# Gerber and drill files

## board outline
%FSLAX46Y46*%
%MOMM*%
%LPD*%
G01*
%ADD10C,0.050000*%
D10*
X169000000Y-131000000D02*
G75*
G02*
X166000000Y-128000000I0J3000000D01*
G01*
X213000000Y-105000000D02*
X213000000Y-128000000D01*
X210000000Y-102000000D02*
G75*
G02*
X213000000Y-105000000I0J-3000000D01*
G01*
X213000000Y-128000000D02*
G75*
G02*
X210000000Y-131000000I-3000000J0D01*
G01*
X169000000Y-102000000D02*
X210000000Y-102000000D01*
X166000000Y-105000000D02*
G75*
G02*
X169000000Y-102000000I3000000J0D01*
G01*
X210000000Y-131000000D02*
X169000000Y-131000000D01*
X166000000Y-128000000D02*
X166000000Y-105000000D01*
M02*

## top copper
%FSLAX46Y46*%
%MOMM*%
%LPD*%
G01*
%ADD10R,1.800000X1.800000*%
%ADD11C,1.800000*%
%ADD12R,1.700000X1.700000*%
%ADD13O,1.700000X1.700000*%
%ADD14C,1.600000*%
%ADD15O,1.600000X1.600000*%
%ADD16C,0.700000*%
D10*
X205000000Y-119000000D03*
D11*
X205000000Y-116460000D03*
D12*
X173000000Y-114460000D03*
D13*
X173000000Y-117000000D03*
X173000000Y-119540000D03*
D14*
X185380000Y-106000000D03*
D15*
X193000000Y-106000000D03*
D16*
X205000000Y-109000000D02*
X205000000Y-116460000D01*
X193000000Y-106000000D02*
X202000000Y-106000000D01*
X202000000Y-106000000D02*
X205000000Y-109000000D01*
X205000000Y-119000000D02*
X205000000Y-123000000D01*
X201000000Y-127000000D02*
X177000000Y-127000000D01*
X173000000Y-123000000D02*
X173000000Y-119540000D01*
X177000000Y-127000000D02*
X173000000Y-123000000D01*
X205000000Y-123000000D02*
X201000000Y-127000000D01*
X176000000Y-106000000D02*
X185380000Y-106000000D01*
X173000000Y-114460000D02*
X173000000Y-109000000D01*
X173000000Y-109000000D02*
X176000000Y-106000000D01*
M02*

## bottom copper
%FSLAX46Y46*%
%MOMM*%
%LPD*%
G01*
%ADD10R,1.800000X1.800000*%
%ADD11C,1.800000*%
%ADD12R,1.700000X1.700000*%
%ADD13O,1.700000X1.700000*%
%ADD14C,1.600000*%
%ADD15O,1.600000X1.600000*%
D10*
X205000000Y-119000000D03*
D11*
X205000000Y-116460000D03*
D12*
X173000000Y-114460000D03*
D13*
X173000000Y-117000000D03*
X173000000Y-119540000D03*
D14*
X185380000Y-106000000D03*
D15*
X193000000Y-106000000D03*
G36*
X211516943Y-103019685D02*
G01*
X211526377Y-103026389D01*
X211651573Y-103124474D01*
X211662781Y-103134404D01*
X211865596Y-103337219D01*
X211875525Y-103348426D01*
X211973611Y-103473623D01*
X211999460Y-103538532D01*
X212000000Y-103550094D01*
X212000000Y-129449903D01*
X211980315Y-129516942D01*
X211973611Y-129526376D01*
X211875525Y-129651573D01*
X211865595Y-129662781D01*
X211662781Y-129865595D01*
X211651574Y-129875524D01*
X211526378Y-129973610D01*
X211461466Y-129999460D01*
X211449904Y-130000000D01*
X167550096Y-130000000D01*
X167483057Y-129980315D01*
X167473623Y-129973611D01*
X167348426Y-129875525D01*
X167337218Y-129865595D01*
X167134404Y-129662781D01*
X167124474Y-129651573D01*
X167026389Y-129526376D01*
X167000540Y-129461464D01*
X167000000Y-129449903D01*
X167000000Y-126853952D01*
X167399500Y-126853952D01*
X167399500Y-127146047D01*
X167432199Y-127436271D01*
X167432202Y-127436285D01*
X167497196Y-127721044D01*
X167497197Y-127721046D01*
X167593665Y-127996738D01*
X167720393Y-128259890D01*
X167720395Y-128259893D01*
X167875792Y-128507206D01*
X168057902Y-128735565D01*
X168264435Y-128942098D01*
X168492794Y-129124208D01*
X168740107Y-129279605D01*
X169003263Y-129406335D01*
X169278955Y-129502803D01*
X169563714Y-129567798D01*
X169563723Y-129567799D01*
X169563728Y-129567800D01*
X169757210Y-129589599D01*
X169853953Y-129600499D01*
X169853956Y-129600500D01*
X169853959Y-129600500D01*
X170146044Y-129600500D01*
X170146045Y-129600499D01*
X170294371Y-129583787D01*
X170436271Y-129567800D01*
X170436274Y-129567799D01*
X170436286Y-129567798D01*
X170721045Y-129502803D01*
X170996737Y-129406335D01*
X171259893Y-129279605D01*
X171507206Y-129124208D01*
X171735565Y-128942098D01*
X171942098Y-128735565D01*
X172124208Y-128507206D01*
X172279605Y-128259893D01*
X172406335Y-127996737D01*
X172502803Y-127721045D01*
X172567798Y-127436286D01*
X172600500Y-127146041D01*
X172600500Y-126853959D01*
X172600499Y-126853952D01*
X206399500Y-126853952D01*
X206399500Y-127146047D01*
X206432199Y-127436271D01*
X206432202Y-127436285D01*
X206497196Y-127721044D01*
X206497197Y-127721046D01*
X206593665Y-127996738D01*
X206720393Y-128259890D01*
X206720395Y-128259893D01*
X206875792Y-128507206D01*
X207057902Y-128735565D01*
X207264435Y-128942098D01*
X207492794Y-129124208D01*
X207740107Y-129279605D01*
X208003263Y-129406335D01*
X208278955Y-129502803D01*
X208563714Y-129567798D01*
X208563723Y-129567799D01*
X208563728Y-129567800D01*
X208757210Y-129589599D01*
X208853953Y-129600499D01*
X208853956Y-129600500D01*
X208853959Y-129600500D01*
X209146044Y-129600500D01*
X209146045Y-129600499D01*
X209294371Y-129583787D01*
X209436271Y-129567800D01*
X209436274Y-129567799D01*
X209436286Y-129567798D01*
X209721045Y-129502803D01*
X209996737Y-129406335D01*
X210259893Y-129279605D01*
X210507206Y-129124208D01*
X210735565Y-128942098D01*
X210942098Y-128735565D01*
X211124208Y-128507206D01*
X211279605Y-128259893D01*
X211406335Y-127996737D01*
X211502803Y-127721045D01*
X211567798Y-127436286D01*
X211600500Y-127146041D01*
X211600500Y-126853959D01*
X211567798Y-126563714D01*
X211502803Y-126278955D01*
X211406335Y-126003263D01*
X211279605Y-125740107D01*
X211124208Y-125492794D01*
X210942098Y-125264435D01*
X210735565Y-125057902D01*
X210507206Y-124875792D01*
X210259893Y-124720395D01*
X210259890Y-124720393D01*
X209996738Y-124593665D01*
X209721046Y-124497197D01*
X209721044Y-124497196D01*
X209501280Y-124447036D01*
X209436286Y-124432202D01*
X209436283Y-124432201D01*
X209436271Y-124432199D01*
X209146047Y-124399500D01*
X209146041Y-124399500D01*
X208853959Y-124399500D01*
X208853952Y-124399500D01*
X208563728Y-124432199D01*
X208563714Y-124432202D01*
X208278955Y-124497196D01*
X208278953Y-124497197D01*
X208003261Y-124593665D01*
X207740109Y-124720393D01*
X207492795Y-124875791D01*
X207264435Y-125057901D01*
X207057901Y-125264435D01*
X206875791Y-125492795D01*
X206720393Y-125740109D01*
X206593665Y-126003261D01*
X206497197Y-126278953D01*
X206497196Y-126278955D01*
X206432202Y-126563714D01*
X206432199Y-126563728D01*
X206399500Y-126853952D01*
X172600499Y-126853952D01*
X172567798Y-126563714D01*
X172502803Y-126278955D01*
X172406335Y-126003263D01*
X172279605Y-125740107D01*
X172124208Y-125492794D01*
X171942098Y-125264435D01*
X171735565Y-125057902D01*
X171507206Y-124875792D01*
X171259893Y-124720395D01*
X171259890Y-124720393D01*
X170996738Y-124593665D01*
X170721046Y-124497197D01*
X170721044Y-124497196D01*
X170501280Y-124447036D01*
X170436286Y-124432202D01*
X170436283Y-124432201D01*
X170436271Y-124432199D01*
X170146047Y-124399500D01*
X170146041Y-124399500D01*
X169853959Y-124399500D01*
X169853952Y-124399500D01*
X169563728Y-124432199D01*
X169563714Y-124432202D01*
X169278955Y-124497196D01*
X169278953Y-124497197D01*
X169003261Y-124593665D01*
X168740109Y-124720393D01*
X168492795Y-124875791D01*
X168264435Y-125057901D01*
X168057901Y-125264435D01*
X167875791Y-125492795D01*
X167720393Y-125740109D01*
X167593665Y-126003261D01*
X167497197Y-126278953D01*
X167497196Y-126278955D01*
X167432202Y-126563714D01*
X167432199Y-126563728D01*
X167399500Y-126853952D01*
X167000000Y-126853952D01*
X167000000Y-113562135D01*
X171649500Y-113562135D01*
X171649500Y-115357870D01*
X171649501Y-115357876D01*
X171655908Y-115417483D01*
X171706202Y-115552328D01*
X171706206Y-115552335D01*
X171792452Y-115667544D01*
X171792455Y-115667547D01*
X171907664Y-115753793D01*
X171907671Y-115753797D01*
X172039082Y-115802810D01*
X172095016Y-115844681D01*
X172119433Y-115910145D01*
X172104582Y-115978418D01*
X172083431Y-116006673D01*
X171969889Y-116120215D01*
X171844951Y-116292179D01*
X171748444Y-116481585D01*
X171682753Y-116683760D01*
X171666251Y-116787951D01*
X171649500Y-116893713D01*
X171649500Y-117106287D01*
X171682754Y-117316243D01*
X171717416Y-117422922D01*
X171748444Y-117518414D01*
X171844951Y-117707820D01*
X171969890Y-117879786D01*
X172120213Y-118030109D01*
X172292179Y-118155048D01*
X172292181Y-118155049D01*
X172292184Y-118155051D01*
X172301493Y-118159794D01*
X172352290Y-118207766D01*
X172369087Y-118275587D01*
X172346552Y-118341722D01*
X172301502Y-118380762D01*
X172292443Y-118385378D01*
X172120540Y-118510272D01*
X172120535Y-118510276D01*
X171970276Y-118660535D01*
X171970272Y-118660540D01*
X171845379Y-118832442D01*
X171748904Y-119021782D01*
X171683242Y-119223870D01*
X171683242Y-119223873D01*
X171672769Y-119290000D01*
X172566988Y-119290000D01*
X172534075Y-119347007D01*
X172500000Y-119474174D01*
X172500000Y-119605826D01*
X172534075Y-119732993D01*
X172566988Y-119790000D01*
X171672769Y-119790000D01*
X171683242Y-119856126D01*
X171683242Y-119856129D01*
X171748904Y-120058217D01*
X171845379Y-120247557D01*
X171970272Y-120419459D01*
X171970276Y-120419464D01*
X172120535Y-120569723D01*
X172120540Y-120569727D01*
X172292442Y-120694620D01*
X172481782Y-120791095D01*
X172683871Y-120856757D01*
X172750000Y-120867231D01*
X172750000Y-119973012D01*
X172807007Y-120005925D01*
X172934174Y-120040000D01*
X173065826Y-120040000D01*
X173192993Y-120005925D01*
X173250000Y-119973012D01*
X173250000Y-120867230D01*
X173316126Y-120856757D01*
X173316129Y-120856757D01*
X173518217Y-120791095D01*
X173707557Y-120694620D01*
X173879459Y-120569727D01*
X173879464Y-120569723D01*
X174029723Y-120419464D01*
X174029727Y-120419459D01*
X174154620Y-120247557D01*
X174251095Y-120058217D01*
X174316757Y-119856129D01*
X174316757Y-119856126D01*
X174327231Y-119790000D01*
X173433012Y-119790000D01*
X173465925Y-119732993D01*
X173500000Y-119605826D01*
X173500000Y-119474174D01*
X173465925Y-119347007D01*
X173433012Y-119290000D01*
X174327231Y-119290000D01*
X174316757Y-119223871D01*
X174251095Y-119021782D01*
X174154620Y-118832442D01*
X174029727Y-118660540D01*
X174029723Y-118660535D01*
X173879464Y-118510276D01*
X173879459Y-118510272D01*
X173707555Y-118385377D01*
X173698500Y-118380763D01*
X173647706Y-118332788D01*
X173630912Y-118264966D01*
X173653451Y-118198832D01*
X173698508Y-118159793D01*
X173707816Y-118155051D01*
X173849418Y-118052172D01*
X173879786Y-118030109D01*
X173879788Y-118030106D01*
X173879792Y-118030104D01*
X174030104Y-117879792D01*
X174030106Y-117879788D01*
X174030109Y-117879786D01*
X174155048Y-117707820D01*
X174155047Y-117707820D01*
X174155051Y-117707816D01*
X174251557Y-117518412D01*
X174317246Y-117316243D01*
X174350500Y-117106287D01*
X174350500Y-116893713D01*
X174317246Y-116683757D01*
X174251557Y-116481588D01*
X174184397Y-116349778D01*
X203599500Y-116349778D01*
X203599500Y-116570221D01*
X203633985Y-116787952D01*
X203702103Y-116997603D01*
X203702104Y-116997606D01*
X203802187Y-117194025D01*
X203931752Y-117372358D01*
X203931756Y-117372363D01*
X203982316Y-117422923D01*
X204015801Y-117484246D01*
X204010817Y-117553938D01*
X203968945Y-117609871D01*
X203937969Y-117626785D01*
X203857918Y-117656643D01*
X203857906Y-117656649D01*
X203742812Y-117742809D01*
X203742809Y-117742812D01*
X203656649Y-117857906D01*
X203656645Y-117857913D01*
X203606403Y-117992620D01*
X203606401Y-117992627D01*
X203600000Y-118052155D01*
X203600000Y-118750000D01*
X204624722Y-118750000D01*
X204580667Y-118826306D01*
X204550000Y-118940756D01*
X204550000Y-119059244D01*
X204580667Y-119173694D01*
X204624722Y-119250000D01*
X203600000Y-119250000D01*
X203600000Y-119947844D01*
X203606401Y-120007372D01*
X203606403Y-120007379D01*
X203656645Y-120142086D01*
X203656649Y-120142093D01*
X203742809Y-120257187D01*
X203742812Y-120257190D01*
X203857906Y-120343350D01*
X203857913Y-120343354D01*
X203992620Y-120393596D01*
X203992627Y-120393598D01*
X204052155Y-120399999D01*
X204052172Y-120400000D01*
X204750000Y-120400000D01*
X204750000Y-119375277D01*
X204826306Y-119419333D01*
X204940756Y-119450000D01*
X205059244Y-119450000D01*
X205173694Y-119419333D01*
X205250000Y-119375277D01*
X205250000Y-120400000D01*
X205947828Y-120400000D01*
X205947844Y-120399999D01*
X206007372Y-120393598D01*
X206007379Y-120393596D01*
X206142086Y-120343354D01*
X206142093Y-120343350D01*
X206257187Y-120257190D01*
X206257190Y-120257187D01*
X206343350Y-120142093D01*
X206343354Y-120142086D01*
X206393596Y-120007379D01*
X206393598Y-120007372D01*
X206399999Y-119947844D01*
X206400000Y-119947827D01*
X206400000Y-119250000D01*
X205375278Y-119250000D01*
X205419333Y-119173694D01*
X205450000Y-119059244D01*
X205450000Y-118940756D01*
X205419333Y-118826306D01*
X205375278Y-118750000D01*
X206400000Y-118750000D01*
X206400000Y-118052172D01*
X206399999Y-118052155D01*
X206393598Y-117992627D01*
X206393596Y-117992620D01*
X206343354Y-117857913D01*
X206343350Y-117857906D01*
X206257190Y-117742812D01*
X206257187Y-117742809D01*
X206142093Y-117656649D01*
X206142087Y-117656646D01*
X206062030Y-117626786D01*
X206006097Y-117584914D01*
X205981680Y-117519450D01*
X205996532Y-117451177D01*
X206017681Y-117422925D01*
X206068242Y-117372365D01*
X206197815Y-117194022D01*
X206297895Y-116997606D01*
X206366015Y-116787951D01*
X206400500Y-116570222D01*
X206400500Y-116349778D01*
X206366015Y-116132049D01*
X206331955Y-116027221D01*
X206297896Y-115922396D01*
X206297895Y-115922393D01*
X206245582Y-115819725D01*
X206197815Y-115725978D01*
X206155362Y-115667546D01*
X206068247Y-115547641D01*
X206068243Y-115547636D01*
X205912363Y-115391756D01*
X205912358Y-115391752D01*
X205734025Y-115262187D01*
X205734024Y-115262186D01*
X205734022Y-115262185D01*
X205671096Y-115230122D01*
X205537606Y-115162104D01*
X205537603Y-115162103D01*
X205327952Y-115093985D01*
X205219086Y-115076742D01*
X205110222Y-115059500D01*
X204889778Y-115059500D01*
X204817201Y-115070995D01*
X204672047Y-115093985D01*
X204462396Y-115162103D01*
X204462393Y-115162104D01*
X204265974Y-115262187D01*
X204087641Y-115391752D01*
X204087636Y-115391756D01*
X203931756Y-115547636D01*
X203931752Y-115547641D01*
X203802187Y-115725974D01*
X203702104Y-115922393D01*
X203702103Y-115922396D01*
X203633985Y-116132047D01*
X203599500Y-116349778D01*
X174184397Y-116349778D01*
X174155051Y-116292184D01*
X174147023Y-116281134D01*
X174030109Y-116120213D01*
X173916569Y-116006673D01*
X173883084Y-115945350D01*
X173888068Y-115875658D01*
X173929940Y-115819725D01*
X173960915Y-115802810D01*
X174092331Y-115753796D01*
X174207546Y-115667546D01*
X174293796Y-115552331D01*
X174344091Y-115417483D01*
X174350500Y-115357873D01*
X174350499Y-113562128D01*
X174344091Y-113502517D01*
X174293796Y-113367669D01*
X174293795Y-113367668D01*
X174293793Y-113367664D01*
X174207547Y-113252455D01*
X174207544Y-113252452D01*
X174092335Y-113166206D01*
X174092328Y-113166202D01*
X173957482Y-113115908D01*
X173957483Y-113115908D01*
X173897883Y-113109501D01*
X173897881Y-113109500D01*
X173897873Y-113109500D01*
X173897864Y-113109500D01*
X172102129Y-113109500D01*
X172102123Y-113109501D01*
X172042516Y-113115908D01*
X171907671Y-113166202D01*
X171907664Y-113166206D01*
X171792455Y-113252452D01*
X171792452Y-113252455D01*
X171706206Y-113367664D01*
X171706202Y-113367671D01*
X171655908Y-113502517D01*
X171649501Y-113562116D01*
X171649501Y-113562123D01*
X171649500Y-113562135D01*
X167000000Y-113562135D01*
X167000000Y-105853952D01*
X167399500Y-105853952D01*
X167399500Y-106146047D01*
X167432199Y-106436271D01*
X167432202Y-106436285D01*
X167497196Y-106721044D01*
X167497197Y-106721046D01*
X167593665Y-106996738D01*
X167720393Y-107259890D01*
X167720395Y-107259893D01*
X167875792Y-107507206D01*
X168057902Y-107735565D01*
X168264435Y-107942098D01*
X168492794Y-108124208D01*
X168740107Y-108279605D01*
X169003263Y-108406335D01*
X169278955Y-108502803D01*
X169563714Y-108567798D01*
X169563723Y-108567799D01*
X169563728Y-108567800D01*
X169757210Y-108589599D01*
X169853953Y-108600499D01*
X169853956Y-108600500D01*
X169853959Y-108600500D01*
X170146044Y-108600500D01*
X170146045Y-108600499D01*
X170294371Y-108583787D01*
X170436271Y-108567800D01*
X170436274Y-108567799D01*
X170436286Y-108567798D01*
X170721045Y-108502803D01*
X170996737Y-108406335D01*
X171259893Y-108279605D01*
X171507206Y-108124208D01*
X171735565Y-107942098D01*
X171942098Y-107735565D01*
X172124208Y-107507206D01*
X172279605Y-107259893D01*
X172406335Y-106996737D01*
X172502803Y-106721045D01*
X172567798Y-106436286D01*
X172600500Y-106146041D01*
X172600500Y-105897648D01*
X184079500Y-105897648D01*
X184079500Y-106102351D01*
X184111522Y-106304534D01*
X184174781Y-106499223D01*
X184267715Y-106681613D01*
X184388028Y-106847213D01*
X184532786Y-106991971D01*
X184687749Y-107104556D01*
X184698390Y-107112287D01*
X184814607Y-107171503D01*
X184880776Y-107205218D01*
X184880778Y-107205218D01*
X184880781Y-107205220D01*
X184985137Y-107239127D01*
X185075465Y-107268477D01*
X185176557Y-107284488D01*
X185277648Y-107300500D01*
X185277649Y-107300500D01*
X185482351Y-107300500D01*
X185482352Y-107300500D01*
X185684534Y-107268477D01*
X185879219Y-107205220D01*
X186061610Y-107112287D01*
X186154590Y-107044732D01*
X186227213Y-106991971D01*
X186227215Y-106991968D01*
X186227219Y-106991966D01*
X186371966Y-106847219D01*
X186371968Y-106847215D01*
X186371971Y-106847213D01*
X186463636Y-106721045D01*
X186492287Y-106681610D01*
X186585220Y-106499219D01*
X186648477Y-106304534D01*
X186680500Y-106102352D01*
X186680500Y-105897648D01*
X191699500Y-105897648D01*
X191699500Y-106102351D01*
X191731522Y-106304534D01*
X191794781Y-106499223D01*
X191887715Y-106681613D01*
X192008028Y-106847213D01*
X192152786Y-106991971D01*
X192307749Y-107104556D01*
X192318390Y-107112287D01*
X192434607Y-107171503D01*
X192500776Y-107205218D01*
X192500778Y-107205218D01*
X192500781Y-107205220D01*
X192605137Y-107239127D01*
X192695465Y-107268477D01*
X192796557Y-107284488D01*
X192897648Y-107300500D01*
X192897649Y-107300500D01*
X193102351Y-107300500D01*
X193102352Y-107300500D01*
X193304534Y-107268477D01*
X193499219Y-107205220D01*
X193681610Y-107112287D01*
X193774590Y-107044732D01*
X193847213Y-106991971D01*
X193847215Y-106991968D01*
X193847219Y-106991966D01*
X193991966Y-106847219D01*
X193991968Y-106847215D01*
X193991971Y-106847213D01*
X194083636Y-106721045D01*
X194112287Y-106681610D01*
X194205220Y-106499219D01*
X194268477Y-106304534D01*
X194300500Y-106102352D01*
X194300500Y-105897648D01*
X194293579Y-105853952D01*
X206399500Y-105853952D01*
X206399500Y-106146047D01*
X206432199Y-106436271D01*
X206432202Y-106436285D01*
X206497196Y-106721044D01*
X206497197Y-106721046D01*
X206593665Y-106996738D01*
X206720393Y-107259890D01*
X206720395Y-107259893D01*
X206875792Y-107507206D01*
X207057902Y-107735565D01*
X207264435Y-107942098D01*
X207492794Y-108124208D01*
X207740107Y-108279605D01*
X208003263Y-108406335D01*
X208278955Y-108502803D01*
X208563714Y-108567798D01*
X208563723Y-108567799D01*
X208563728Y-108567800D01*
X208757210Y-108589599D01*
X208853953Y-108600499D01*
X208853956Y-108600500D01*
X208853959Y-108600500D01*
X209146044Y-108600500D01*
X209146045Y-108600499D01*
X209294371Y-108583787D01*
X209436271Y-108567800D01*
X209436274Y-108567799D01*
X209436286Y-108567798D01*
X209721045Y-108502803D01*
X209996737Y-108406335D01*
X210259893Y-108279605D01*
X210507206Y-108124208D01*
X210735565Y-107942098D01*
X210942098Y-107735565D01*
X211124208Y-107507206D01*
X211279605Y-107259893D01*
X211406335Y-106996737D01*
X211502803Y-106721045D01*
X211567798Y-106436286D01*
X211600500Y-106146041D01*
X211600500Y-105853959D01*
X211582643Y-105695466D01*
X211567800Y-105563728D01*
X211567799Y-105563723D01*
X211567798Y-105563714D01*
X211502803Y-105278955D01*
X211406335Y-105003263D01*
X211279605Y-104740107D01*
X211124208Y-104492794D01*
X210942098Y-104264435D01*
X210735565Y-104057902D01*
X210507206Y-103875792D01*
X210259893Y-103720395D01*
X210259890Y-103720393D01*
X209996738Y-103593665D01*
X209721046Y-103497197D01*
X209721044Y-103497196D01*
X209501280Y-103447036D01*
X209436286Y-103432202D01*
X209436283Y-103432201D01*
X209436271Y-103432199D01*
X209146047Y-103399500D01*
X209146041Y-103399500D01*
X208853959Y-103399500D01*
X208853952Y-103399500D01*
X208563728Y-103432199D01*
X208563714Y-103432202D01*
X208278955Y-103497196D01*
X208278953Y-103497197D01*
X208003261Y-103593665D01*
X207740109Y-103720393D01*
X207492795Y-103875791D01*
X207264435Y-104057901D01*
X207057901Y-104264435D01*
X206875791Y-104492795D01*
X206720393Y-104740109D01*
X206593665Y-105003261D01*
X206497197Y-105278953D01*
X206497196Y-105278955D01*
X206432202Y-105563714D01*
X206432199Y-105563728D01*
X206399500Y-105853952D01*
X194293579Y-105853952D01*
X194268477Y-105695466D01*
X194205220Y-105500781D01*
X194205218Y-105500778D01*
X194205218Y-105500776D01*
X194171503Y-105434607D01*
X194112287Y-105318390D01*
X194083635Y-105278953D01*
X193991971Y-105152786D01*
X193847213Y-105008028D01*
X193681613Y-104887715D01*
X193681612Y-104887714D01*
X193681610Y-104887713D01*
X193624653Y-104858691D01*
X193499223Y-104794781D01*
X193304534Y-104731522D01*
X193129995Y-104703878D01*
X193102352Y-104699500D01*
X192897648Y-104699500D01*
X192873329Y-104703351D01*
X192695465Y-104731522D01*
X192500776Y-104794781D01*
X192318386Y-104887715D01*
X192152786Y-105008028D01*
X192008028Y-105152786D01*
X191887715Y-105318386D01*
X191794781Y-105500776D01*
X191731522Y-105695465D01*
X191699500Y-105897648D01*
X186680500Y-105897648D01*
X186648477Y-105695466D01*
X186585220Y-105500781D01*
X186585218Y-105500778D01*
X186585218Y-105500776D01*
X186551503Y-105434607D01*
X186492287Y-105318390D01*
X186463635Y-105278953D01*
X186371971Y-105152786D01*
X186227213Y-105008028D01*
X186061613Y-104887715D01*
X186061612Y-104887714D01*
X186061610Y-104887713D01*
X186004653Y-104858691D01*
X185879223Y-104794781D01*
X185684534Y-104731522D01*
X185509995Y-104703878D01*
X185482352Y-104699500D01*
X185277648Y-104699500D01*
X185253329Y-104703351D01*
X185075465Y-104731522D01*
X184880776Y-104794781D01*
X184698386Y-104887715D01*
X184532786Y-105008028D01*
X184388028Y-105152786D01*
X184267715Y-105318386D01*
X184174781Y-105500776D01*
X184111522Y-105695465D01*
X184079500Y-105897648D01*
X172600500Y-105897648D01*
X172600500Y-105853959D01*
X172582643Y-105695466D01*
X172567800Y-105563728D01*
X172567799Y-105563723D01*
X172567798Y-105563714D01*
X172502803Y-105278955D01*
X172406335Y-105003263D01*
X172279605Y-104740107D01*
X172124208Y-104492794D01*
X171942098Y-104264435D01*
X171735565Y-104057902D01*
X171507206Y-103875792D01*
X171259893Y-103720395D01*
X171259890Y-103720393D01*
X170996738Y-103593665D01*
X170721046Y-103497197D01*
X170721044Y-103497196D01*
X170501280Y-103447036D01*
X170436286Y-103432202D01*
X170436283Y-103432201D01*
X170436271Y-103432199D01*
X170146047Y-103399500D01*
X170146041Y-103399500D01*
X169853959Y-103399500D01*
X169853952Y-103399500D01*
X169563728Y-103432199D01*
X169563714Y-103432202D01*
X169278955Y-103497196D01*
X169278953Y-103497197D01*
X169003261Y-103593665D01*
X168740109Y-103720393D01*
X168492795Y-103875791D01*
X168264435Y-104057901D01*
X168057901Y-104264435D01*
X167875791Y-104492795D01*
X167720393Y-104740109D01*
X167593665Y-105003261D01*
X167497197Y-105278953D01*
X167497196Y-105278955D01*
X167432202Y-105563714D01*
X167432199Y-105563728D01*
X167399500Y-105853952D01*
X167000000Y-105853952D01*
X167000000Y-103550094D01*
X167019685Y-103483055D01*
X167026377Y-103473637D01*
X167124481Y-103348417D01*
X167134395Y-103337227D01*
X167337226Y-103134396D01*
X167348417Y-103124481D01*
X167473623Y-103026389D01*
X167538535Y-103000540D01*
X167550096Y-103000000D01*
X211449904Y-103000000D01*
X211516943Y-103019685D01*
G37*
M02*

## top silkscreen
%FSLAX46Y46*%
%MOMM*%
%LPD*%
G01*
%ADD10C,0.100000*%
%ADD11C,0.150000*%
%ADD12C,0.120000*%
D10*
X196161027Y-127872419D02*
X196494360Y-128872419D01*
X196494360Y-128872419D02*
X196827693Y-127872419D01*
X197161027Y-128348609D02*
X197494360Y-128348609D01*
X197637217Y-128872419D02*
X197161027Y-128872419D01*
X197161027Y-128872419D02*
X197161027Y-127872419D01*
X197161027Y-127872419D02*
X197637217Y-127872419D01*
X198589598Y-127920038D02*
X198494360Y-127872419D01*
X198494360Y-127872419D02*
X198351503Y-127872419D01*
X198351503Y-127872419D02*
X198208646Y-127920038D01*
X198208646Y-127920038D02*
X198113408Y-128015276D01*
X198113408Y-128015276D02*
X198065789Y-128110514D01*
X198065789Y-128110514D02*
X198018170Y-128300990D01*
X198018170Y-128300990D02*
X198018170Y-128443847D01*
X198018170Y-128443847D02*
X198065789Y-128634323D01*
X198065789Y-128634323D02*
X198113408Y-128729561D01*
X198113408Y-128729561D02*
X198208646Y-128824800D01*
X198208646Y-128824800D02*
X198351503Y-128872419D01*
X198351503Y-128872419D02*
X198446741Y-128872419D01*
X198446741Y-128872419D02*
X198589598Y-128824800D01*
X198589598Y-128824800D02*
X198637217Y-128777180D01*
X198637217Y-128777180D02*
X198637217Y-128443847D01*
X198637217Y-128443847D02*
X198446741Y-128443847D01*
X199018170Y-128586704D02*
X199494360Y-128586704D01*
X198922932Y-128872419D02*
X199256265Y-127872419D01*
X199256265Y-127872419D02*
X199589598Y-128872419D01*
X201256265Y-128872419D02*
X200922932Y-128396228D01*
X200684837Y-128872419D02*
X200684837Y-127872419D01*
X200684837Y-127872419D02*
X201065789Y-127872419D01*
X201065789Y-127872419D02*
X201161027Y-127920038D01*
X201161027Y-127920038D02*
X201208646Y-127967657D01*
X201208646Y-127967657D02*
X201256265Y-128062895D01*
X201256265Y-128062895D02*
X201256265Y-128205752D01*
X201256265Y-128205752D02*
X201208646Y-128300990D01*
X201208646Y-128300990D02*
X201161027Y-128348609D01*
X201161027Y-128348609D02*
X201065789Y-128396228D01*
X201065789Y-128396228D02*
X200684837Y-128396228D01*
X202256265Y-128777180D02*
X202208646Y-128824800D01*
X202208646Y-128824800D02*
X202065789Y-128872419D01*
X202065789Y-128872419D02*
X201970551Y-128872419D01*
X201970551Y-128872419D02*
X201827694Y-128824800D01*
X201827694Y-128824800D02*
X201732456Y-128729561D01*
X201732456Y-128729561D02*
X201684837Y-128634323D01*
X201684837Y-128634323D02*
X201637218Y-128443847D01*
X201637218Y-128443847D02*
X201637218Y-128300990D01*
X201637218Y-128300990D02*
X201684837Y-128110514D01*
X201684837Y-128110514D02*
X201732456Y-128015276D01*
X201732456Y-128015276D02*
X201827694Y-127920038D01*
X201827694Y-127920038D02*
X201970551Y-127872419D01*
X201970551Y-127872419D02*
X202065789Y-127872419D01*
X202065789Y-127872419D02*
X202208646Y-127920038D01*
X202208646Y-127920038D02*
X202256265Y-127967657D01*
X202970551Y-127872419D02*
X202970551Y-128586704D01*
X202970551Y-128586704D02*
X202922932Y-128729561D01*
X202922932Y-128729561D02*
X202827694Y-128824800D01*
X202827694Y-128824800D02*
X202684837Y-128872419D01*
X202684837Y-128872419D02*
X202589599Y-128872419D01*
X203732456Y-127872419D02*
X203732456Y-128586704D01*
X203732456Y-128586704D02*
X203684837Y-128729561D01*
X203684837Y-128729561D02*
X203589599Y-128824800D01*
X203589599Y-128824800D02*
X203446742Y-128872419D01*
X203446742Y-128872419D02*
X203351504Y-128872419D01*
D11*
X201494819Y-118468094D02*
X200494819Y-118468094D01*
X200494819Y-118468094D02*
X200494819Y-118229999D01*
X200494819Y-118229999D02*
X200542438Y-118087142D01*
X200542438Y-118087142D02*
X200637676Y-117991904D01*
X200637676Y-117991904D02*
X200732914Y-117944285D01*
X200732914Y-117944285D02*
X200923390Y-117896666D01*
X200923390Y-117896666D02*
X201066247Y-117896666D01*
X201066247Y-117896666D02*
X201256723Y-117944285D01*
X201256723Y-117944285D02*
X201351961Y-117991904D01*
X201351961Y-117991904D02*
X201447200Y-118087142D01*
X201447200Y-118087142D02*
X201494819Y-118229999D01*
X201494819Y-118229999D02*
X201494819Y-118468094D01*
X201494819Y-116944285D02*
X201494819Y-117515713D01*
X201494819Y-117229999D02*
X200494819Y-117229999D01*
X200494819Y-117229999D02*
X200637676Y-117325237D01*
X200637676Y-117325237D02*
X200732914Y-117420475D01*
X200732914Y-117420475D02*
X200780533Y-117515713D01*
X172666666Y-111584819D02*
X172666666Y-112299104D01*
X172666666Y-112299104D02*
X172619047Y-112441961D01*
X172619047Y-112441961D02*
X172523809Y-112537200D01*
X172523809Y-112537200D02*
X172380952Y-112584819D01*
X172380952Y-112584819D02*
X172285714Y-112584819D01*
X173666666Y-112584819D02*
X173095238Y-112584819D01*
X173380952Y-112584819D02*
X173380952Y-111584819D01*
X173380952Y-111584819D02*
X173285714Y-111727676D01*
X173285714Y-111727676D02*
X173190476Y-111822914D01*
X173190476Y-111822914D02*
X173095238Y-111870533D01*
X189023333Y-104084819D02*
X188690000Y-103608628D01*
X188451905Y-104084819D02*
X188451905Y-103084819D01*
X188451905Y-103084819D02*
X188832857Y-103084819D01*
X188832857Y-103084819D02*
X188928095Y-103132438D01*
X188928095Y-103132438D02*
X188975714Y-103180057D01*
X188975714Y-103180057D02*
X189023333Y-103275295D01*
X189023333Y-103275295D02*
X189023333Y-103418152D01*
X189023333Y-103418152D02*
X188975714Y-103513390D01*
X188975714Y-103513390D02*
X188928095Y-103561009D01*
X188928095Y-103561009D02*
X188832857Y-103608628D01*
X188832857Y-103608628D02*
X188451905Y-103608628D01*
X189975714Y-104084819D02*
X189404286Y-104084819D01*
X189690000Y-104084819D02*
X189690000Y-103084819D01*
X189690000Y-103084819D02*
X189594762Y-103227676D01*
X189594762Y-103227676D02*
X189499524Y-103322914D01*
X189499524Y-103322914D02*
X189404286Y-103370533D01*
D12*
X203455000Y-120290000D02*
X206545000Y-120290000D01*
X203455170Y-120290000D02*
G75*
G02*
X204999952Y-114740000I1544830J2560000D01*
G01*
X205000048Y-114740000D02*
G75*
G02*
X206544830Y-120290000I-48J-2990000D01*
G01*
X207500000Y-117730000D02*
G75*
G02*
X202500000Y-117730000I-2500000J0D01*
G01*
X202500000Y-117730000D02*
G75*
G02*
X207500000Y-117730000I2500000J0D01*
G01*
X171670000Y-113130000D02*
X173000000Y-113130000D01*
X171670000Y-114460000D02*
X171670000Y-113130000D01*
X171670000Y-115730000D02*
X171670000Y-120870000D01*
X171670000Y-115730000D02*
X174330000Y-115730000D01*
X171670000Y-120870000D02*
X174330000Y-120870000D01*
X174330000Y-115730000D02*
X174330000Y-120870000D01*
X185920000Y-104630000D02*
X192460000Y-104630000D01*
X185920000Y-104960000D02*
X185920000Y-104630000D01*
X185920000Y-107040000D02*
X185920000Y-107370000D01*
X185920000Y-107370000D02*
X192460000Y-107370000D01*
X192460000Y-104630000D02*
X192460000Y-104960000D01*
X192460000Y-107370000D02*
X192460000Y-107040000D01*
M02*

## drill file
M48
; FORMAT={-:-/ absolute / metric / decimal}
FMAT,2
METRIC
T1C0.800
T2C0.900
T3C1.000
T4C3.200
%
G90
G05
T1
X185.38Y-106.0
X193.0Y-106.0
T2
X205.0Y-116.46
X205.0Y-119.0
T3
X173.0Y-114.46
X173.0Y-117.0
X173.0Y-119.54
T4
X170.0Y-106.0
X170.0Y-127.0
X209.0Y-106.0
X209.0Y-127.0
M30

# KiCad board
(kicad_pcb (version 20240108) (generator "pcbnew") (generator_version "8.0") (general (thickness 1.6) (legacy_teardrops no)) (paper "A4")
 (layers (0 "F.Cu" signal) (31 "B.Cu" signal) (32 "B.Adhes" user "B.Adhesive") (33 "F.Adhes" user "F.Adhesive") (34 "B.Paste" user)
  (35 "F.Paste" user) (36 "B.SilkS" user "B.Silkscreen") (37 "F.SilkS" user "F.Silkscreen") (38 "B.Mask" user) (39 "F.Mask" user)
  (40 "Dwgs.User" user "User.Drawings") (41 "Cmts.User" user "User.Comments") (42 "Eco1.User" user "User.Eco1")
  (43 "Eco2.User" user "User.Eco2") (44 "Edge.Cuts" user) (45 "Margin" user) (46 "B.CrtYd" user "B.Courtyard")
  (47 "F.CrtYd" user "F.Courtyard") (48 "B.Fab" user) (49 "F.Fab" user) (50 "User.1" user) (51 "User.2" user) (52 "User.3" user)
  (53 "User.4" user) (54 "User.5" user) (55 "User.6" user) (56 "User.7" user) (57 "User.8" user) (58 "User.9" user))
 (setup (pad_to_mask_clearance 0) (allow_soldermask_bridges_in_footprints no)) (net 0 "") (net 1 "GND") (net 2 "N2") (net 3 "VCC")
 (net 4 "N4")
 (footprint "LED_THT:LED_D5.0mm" (layer "F.Cu") (at 205 119 90)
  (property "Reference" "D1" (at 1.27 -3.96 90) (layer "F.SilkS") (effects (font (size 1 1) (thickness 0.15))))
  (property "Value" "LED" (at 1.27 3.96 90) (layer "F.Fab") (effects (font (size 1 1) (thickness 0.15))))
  (fp_line (start -1.29 -1.545) (end -1.29 1.545) (stroke (width 0.12) (type solid)) (layer "F.SilkS"))
  (fp_arc (start -1.29 -1.54483) (mid 2.071756 -2.880501) (end 4.26 -0.000048) (stroke (width 0.12) (type solid)) (layer "F.SilkS"))
  (fp_arc (start 4.26 0.000048) (mid 2.071756 2.880501) (end -1.29 1.54483) (stroke (width 0.12) (type solid)) (layer "F.SilkS"))
  (fp_circle (center 1.27 0) (end 3.77 0) (stroke (width 0.12) (type solid)) (fill none) (layer "F.SilkS"))
  (pad "1" thru_hole rect (at 0 0 90) (size 1.8 1.8) (drill 0.9) (layers "*.Cu" "*.Mask") (remove_unused_layers no) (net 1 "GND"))
  (pad "2" thru_hole circle (at 2.54 0 90) (size 1.8 1.8) (drill 0.9) (layers "*.Cu" "*.Mask") (remove_unused_layers no) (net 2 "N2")))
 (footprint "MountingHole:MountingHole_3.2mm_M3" (layer "F.Cu") (at 209 106)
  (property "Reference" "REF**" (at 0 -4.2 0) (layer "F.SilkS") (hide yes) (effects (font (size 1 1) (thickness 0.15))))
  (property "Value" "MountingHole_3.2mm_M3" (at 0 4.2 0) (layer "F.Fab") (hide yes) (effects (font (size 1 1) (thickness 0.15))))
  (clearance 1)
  (pad "" np_thru_hole circle (at 0 0) (size 3.2 3.2) (drill 3.2) (layers "*.Cu" "*.Mask")))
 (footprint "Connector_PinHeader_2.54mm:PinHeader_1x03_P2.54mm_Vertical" (layer "F.Cu") (at 173 114.46)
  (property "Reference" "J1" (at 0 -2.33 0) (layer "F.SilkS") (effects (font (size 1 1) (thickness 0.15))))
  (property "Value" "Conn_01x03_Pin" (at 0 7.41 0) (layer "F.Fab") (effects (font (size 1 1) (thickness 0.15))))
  (fp_line (start -1.33 -1.33) (end 0 -1.33) (stroke (width 0.12) (type solid)) (layer "F.SilkS"))
  (fp_line (start -1.33 0) (end -1.33 -1.33) (stroke (width 0.12) (type solid)) (layer "F.SilkS"))
  (fp_line (start -1.33 1.27) (end -1.33 6.41) (stroke (width 0.12) (type solid)) (layer "F.SilkS"))
  (fp_line (start -1.33 1.27) (end 1.33 1.27) (stroke (width 0.12) (type solid)) (layer "F.SilkS"))
  (fp_line (start -1.33 6.41) (end 1.33 6.41) (stroke (width 0.12) (type solid)) (layer "F.SilkS"))
  (fp_line (start 1.33 1.27) (end 1.33 6.41) (stroke (width 0.12) (type solid)) (layer "F.SilkS"))
  (pad "1" thru_hole rect (at 0 0) (size 1.7 1.7) (drill 1) (layers "*.Cu" "*.Mask") (remove_unused_layers no) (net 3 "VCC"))
  (pad "2" thru_hole oval (at 0 2.54) (size 1.7 1.7) (drill 1) (layers "*.Cu" "*.Mask") (remove_unused_layers no) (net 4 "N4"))
  (pad "3" thru_hole oval (at 0 5.08) (size 1.7 1.7) (drill 1) (layers "*.Cu" "*.Mask") (remove_unused_layers no) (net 1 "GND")))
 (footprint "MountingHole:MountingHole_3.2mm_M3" (layer "F.Cu") (at 170 127)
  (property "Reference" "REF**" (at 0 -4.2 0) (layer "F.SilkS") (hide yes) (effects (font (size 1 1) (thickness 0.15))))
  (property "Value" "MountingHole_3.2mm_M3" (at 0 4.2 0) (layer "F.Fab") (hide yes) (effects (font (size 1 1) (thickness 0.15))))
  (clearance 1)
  (pad "" np_thru_hole circle (at 0 0) (size 3.2 3.2) (drill 3.2) (layers "*.Cu" "*.Mask")))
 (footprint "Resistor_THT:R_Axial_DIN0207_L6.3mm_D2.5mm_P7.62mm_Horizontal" (layer "F.Cu") (at 185.38 106)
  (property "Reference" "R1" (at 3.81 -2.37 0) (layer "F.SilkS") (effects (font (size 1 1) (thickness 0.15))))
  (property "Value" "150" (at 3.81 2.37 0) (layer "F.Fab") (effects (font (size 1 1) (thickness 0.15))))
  (fp_line (start 0.54 -1.37) (end 7.08 -1.37) (stroke (width 0.12) (type solid)) (layer "F.SilkS"))
  (fp_line (start 0.54 -1.04) (end 0.54 -1.37) (stroke (width 0.12) (type solid)) (layer "F.SilkS"))
  (fp_line (start 0.54 1.04) (end 0.54 1.37) (stroke (width 0.12) (type solid)) (layer "F.SilkS"))
  (fp_line (start 0.54 1.37) (end 7.08 1.37) (stroke (width 0.12) (type solid)) (layer "F.SilkS"))
  (fp_line (start 7.08 -1.37) (end 7.08 -1.04) (stroke (width 0.12) (type solid)) (layer "F.SilkS"))
  (fp_line (start 7.08 1.37) (end 7.08 1.04) (stroke (width 0.12) (type solid)) (layer "F.SilkS"))
  (pad "1" thru_hole circle (at 0 0) (size 1.6 1.6) (drill 0.8) (layers "*.Cu" "*.Mask") (remove_unused_layers no) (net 3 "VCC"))
  (pad "2" thru_hole oval (at 7.62 0) (size 1.6 1.6) (drill 0.8) (layers "*.Cu" "*.Mask") (remove_unused_layers no) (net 2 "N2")))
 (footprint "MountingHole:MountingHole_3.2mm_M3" (layer "F.Cu") (at 209 127)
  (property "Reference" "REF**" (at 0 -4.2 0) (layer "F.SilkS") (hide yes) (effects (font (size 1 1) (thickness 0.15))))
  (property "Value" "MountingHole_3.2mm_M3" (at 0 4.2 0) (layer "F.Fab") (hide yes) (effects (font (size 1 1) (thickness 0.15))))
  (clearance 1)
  (pad "" np_thru_hole circle (at 0 0) (size 3.2 3.2) (drill 3.2) (layers "*.Cu" "*.Mask")))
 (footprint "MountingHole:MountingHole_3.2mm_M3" (layer "F.Cu") (at 170 106)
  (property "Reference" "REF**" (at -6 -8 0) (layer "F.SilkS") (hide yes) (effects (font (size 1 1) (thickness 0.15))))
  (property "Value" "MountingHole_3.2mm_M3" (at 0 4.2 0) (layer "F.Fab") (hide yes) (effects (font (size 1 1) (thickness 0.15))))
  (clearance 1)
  (pad "" np_thru_hole circle (at 0 0) (size 3.2 3.2) (drill 3.2) (layers "*.Cu" "*.Mask")))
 (gr_arc (start 169 131) (mid 166.87868 130.12132) (end 166 128) (stroke (width 0.05) (type default)) (layer "Edge.Cuts"))
 (gr_line (start 213 105) (end 213 128) (stroke (width 0.05) (type default)) (layer "Edge.Cuts"))
 (gr_arc (start 210 102) (mid 212.12132 102.87868) (end 213 105) (stroke (width 0.05) (type default)) (layer "Edge.Cuts"))
 (gr_arc (start 213 128) (mid 212.12132 130.12132) (end 210 131) (stroke (width 0.05) (type default)) (layer "Edge.Cuts"))
 (gr_line (start 169 102) (end 210 102) (stroke (width 0.05) (type default)) (layer "Edge.Cuts"))
 (gr_arc (start 166 105) (mid 166.87868 102.87868) (end 169 102) (stroke (width 0.05) (type default)) (layer "Edge.Cuts"))
 (gr_line (start 210 131) (end 169 131) (stroke (width 0.05) (type default)) (layer "Edge.Cuts"))
 (gr_line (start 166 128) (end 166 105) (stroke (width 0.05) (type default)) (layer "Edge.Cuts"))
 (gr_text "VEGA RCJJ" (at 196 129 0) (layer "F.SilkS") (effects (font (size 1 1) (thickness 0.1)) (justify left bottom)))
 (segment (start 205 109) (end 205 116.46) (width 0.7) (layer "F.Cu") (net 2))
 (segment (start 193 106) (end 202 106) (width 0.7) (layer "F.Cu") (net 2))
 (segment (start 202 106) (end 205 109) (width 0.7) (layer "F.Cu") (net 2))
 (segment (start 205 119) (end 205 123) (width 0.7) (layer "F.Cu") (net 1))
 (segment (start 201 127) (end 177 127) (width 0.7) (layer "F.Cu") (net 1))
 (segment (start 173 123) (end 173 119.54) (width 0.7) (layer "F.Cu") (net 1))
 (segment (start 177 127) (end 173 123) (width 0.7) (layer "F.Cu") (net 1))
 (segment (start 205 123) (end 201 127) (width 0.7) (layer "F.Cu") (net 1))
 (segment (start 176 106) (end 185.38 106) (width 0.7) (layer "F.Cu") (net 3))
 (segment (start 173 114.46) (end 173 109) (width 0.7) (layer "F.Cu") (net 3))
 (segment (start 173 109) (end 176 106) (width 0.7) (layer "F.Cu") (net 3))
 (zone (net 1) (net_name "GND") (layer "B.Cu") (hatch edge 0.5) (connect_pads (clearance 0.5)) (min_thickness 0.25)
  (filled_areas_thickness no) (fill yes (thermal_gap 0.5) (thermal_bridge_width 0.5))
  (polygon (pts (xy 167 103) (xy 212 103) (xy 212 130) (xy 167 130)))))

